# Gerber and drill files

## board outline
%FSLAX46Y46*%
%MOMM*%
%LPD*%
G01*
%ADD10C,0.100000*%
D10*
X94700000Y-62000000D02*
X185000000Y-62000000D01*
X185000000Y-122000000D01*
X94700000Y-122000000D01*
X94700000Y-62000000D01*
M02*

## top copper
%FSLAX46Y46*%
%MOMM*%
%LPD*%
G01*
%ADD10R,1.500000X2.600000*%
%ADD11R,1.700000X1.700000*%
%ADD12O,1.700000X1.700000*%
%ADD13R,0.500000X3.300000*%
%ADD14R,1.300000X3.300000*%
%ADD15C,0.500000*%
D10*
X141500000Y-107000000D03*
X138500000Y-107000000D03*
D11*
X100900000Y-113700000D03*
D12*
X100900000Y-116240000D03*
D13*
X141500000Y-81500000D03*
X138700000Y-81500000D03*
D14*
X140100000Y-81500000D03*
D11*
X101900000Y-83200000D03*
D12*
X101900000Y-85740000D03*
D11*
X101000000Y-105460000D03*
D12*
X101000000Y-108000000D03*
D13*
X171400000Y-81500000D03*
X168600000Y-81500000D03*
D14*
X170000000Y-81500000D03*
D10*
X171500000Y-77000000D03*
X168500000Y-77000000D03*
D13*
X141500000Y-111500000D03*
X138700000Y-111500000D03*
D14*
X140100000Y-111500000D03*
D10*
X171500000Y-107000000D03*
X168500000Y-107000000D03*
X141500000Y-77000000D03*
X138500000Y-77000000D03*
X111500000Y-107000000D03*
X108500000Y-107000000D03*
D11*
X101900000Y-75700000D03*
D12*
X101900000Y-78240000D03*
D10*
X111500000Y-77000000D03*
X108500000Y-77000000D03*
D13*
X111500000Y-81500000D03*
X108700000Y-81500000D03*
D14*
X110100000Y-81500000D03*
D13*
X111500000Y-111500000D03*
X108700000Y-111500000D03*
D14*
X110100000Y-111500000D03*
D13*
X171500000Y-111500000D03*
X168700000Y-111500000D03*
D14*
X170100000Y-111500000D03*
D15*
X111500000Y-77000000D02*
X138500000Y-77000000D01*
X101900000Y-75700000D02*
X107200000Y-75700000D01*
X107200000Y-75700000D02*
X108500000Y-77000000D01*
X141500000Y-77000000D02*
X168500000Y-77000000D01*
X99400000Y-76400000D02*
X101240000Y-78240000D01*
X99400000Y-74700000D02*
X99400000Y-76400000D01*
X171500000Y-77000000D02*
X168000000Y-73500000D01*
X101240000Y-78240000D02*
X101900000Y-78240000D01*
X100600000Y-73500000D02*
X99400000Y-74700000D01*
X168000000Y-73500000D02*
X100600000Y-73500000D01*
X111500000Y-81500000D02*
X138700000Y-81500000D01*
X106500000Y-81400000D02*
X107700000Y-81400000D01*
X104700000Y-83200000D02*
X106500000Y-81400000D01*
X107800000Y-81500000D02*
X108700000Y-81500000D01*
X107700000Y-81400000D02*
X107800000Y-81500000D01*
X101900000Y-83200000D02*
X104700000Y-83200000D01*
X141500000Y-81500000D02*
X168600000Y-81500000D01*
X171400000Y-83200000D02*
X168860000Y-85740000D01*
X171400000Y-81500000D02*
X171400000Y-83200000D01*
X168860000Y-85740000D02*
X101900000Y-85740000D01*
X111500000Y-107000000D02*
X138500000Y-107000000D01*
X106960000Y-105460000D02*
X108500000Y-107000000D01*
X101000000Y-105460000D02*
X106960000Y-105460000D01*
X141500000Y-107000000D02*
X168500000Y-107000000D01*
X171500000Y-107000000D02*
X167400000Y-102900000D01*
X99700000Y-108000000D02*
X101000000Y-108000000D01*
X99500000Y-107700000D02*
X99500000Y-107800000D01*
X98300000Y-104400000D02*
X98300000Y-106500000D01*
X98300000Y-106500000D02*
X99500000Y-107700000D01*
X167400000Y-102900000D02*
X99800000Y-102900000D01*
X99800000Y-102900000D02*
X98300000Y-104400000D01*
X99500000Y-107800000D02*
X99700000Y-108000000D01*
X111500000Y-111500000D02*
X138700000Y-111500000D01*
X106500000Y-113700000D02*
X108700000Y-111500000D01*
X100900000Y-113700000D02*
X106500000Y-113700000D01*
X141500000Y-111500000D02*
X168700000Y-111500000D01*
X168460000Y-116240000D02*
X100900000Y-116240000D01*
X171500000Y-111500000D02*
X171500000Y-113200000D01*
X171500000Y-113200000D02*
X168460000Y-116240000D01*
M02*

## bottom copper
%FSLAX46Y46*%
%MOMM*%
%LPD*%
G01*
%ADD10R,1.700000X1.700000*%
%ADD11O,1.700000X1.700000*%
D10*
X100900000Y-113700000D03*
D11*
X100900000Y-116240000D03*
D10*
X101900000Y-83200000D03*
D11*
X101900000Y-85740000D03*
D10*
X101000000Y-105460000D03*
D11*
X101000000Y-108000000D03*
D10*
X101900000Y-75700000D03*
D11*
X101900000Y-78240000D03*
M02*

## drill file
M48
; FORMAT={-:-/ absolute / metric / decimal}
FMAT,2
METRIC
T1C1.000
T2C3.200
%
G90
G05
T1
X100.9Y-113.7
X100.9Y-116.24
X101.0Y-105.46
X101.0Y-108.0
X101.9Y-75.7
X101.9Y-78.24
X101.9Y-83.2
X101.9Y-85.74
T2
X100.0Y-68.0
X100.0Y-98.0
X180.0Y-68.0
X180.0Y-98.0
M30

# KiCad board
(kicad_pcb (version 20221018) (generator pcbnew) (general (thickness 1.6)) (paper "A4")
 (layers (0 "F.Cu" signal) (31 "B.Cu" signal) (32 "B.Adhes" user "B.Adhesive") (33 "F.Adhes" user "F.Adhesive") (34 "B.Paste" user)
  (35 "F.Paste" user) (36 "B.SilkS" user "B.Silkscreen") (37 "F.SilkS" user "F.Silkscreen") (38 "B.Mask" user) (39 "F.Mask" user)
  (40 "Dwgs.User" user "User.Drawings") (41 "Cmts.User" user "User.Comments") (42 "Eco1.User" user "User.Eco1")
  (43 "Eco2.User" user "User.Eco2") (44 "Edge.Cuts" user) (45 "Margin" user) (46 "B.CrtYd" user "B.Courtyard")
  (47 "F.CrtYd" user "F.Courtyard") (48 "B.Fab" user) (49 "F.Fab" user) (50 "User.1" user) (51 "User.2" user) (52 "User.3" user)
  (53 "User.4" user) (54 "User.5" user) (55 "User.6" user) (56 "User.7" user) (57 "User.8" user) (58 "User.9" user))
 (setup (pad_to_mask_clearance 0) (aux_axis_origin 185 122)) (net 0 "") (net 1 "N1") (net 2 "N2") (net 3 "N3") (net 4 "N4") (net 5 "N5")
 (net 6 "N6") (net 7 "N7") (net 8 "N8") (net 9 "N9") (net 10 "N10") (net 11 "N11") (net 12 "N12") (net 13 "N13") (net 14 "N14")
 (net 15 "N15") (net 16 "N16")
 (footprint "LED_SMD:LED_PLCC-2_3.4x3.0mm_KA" (layer "F.Cu") (at 140 107 180)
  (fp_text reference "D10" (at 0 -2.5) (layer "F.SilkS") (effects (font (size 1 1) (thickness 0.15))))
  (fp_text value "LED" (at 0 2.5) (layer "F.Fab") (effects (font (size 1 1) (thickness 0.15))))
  (pad "1" smd rect (at -1.5 0 180) (size 1.5 2.6) (layers "F.Cu" "F.Paste" "F.Mask") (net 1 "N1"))
  (pad "2" smd rect (at 1.5 0 180) (size 1.5 2.6) (layers "F.Cu" "F.Paste" "F.Mask") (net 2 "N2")))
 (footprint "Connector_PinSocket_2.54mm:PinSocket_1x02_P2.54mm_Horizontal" (layer "F.Cu") (at 100.9 113.7)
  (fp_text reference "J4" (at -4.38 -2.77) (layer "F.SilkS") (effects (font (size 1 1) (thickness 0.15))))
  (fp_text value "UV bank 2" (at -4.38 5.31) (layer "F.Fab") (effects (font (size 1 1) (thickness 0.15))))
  (pad "1" thru_hole rect (at 0 0) (size 1.7 1.7) (drill 1) (layers "*.Cu" "*.Mask") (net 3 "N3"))
  (pad "2" thru_hole oval (at 0 2.54) (size 1.7 1.7) (drill 1) (layers "*.Cu" "*.Mask") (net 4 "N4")))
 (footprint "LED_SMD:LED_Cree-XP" (layer "F.Cu") (at 140.1 81.5 180)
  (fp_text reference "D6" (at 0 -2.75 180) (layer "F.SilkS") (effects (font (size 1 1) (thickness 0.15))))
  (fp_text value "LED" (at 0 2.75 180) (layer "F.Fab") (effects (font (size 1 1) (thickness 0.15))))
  (pad "" smd rect (at 0 -1 180) (size 1.01 0.75) (layers "F.Paste"))
  (pad "" smd rect (at 0 0 180) (size 1.01 0.75) (layers "F.Paste"))
  (pad "" smd rect (at 0 1 180) (size 1.01 0.75) (layers "F.Paste"))
  (pad "1" smd rect (at -1.4 0 180) (size 0.5 3.3) (layers "F.Cu" "F.Paste" "F.Mask") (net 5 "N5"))
  (pad "2" smd rect (at 1.4 0 180) (size 0.5 3.3) (layers "F.Cu" "F.Paste" "F.Mask") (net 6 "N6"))
  (pad "3" smd rect (at 0 0 180) (size 1.3 3.3) (layers "F.Cu" "F.Mask")))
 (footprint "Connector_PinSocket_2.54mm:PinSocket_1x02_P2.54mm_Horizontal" (layer "F.Cu") (at 101.9 83.2)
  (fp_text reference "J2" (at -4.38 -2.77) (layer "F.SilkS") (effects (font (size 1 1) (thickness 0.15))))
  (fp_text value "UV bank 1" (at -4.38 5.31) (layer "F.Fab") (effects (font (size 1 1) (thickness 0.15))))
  (pad "1" thru_hole rect (at 0 0) (size 1.7 1.7) (drill 1) (layers "*.Cu" "*.Mask") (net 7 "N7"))
  (pad "2" thru_hole oval (at 0 2.54) (size 1.7 1.7) (drill 1) (layers "*.Cu" "*.Mask") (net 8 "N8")))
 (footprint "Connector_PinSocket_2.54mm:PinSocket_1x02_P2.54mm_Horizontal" (layer "F.Cu") (at 101 105.46)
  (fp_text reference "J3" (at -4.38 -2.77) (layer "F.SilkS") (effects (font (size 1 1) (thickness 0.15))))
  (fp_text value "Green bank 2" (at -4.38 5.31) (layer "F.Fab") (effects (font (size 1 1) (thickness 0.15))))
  (pad "1" thru_hole rect (at 0 0) (size 1.7 1.7) (drill 1) (layers "*.Cu" "*.Mask") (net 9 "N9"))
  (pad "2" thru_hole oval (at 0 2.54) (size 1.7 1.7) (drill 1) (layers "*.Cu" "*.Mask") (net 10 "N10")))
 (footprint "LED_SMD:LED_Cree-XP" (layer "F.Cu") (at 170 81.5 180)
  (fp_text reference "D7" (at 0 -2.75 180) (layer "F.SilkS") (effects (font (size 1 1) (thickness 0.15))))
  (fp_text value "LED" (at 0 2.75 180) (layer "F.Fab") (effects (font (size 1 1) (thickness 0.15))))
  (pad "" smd rect (at 0 -1 180) (size 1.01 0.75) (layers "F.Paste"))
  (pad "" smd rect (at 0 0 180) (size 1.01 0.75) (layers "F.Paste"))
  (pad "" smd rect (at 0 1 180) (size 1.01 0.75) (layers "F.Paste"))
  (pad "1" smd rect (at -1.4 0 180) (size 0.5 3.3) (layers "F.Cu" "F.Paste" "F.Mask") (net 8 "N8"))
  (pad "2" smd rect (at 1.4 0 180) (size 0.5 3.3) (layers "F.Cu" "F.Paste" "F.Mask") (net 5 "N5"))
  (pad "3" smd rect (at 0 0 180) (size 1.3 3.3) (layers "F.Cu" "F.Mask")))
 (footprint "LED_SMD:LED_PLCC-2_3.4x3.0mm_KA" (layer "F.Cu") (at 170 77 180)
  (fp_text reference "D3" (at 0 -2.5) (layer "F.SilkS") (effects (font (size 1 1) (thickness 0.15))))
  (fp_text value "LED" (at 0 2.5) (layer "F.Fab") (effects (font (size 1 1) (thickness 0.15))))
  (pad "1" smd rect (at -1.5 0 180) (size 1.5 2.6) (layers "F.Cu" "F.Paste" "F.Mask") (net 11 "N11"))
  (pad "2" smd rect (at 1.5 0 180) (size 1.5 2.6) (layers "F.Cu" "F.Paste" "F.Mask") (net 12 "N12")))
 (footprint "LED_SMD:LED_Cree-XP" (layer "F.Cu") (at 140.1 111.5 180)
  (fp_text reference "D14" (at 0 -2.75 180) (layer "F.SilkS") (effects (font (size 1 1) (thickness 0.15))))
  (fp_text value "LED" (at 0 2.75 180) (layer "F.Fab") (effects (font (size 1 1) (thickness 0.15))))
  (pad "" smd rect (at 0 -1 180) (size 1.01 0.75) (layers "F.Paste"))
  (pad "" smd rect (at 0 0 180) (size 1.01 0.75) (layers "F.Paste"))
  (pad "" smd rect (at 0 1 180) (size 1.01 0.75) (layers "F.Paste"))
  (pad "1" smd rect (at -1.4 0 180) (size 0.5 3.3) (layers "F.Cu" "F.Paste" "F.Mask") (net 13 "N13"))
  (pad "2" smd rect (at 1.4 0 180) (size 0.5 3.3) (layers "F.Cu" "F.Paste" "F.Mask") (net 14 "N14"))
  (pad "3" smd rect (at 0 0 180) (size 1.3 3.3) (layers "F.Cu" "F.Mask")))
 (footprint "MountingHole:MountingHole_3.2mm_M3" (layer "F.Cu") (at 180 68)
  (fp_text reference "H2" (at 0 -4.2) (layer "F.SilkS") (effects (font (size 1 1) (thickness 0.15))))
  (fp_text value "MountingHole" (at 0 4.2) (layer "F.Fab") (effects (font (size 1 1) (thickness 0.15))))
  (pad "" np_thru_hole circle (at 0 0) (size 3.2 3.2) (drill 3.2) (layers "*.Cu" "*.Mask")))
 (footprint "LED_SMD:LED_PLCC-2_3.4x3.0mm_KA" (layer "F.Cu") (at 170 107 180)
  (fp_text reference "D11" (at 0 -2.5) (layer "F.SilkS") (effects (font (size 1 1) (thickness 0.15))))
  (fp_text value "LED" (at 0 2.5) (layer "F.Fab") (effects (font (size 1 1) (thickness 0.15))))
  (pad "1" smd rect (at -1.5 0 180) (size 1.5 2.6) (layers "F.Cu" "F.Paste" "F.Mask") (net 10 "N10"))
  (pad "2" smd rect (at 1.5 0 180) (size 1.5 2.6) (layers "F.Cu" "F.Paste" "F.Mask") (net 1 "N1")))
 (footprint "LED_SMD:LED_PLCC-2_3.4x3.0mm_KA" (layer "F.Cu") (at 140 77 180)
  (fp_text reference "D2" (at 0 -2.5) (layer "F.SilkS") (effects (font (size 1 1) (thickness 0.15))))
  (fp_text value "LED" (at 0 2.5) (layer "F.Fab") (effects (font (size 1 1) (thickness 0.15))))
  (pad "1" smd rect (at -1.5 0 180) (size 1.5 2.6) (layers "F.Cu" "F.Paste" "F.Mask") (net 12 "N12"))
  (pad "2" smd rect (at 1.5 0 180) (size 1.5 2.6) (layers "F.Cu" "F.Paste" "F.Mask") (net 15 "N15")))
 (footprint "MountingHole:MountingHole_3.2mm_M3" (layer "F.Cu") (at 100 98)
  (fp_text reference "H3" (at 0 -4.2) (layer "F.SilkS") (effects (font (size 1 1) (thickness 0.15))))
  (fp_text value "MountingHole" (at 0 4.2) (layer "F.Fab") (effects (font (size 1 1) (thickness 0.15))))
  (pad "" np_thru_hole circle (at 0 0) (size 3.2 3.2) (drill 3.2) (layers "*.Cu" "*.Mask")))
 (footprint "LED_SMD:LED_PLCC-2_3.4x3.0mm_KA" (layer "F.Cu") (at 110 107 180)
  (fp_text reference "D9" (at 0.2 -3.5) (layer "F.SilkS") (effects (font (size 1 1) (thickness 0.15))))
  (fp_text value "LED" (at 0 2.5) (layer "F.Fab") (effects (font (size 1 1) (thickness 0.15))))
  (pad "1" smd rect (at -1.5 0 180) (size 1.5 2.6) (layers "F.Cu" "F.Paste" "F.Mask") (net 2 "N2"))
  (pad "2" smd rect (at 1.5 0 180) (size 1.5 2.6) (layers "F.Cu" "F.Paste" "F.Mask") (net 9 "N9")))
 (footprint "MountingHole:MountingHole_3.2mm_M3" (layer "F.Cu") (at 180 98)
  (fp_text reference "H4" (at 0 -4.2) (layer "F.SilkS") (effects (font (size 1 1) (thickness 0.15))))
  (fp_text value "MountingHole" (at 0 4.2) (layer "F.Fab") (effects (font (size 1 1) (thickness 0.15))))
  (pad "" np_thru_hole circle (at 0 0) (size 3.2 3.2) (drill 3.2) (layers "*.Cu" "*.Mask")))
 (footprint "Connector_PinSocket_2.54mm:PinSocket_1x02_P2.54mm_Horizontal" (layer "F.Cu") (at 101.9 75.7)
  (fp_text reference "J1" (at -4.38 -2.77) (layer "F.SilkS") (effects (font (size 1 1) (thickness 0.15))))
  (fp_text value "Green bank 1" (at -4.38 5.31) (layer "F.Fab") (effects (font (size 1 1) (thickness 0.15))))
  (pad "1" thru_hole rect (at 0 0) (size 1.7 1.7) (drill 1) (layers "*.Cu" "*.Mask") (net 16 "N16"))
  (pad "2" thru_hole oval (at 0 2.54) (size 1.7 1.7) (drill 1) (layers "*.Cu" "*.Mask") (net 11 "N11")))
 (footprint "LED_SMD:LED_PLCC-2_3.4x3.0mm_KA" (layer "F.Cu") (at 110 77 180)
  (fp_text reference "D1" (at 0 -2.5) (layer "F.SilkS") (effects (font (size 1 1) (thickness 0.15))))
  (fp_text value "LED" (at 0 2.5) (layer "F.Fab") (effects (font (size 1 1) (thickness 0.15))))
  (pad "1" smd rect (at -1.5 0 180) (size 1.5 2.6) (layers "F.Cu" "F.Paste" "F.Mask") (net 15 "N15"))
  (pad "2" smd rect (at 1.5 0 180) (size 1.5 2.6) (layers "F.Cu" "F.Paste" "F.Mask") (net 16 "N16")))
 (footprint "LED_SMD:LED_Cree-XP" (layer "F.Cu") (at 110.1 81.5 180)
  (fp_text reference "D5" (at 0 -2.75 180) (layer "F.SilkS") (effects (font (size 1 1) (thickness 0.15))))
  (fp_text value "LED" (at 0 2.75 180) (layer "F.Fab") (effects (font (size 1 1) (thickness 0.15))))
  (pad "" smd rect (at 0 -1 180) (size 1.01 0.75) (layers "F.Paste"))
  (pad "" smd rect (at 0 0 180) (size 1.01 0.75) (layers "F.Paste"))
  (pad "" smd rect (at 0 1 180) (size 1.01 0.75) (layers "F.Paste"))
  (pad "1" smd rect (at -1.4 0 180) (size 0.5 3.3) (layers "F.Cu" "F.Paste" "F.Mask") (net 6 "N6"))
  (pad "2" smd rect (at 1.4 0 180) (size 0.5 3.3) (layers "F.Cu" "F.Paste" "F.Mask") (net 7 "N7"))
  (pad "3" smd rect (at 0 0 180) (size 1.3 3.3) (layers "F.Cu" "F.Mask")))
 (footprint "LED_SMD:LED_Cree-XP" (layer "F.Cu") (at 110.1 111.5 180)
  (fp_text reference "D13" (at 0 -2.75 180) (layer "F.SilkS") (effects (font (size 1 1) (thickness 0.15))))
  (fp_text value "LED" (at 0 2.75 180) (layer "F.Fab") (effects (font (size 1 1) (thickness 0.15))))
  (pad "" smd rect (at 0 -1 180) (size 1.01 0.75) (layers "F.Paste"))
  (pad "" smd rect (at 0 0 180) (size 1.01 0.75) (layers "F.Paste"))
  (pad "" smd rect (at 0 1 180) (size 1.01 0.75) (layers "F.Paste"))
  (pad "1" smd rect (at -1.4 0 180) (size 0.5 3.3) (layers "F.Cu" "F.Paste" "F.Mask") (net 14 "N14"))
  (pad "2" smd rect (at 1.4 0 180) (size 0.5 3.3) (layers "F.Cu" "F.Paste" "F.Mask") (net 3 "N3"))
  (pad "3" smd rect (at 0 0 180) (size 1.3 3.3) (layers "F.Cu" "F.Mask")))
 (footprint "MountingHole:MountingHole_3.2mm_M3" (layer "F.Cu") (at 100 68)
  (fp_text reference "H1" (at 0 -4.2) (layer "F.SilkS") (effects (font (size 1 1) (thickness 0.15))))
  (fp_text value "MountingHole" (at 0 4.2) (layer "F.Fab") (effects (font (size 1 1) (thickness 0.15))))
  (pad "" np_thru_hole circle (at 0 0) (size 3.2 3.2) (drill 3.2) (layers "*.Cu" "*.Mask")))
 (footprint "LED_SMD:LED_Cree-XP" (layer "F.Cu") (at 170.1 111.5 180)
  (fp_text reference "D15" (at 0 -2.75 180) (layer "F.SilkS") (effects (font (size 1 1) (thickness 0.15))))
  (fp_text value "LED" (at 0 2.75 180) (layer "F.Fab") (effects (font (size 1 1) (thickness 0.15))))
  (pad "" smd rect (at 0 -1 180) (size 1.01 0.75) (layers "F.Paste"))
  (pad "" smd rect (at 0 0 180) (size 1.01 0.75) (layers "F.Paste"))
  (pad "" smd rect (at 0 1 180) (size 1.01 0.75) (layers "F.Paste"))
  (pad "1" smd rect (at -1.4 0 180) (size 0.5 3.3) (layers "F.Cu" "F.Paste" "F.Mask") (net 4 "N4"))
  (pad "2" smd rect (at 1.4 0 180) (size 0.5 3.3) (layers "F.Cu" "F.Paste" "F.Mask") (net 13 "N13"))
  (pad "3" smd rect (at 0 0 180) (size 1.3 3.3) (layers "F.Cu" "F.Mask")))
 (gr_rect (start 94.7 62) (end 185 122) (stroke (width 0.1) (type default)) (fill none) (layer "Edge.Cuts"))
 (segment (start 111.5 77) (end 138.5 77) (width 0.5) (layer "F.Cu") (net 15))
 (segment (start 101.9 75.7) (end 107.2 75.7) (width 0.5) (layer "F.Cu") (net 16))
 (segment (start 107.2 75.7) (end 108.5 77) (width 0.5) (layer "F.Cu") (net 16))
 (segment (start 141.5 77) (end 168.5 77) (width 0.5) (layer "F.Cu") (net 12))
 (segment (start 99.4 76.4) (end 101.24 78.24) (width 0.5) (layer "F.Cu") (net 11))
 (segment (start 99.4 74.7) (end 99.4 76.4) (width 0.5) (layer "F.Cu") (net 11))
 (segment (start 171.5 77) (end 168 73.5) (width 0.5) (layer "F.Cu") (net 11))
 (segment (start 101.24 78.24) (end 101.9 78.24) (width 0.5) (layer "F.Cu") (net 11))
 (segment (start 100.6 73.5) (end 99.4 74.7) (width 0.5) (layer "F.Cu") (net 11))
 (segment (start 168 73.5) (end 100.6 73.5) (width 0.5) (layer "F.Cu") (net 11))
 (segment (start 111.5 81.5) (end 138.7 81.5) (width 0.5) (layer "F.Cu") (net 6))
 (segment (start 106.5 81.4) (end 107.7 81.4) (width 0.5) (layer "F.Cu") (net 7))
 (segment (start 104.7 83.2) (end 106.5 81.4) (width 0.5) (layer "F.Cu") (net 7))
 (segment (start 107.8 81.5) (end 108.7 81.5) (width 0.5) (layer "F.Cu") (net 7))
 (segment (start 107.7 81.4) (end 107.8 81.5) (width 0.5) (layer "F.Cu") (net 7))
 (segment (start 101.9 83.2) (end 104.7 83.2) (width 0.5) (layer "F.Cu") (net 7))
 (segment (start 141.5 81.5) (end 168.6 81.5) (width 0.5) (layer "F.Cu") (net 5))
 (segment (start 171.4 83.2) (end 168.86 85.74) (width 0.5) (layer "F.Cu") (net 8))
 (segment (start 171.4 81.5) (end 171.4 83.2) (width 0.5) (layer "F.Cu") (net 8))
 (segment (start 168.86 85.74) (end 101.9 85.74) (width 0.5) (layer "F.Cu") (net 8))
 (segment (start 111.5 107) (end 138.5 107) (width 0.5) (layer "F.Cu") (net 2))
 (segment (start 106.96 105.46) (end 108.5 107) (width 0.5) (layer "F.Cu") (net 9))
 (segment (start 101 105.46) (end 106.96 105.46) (width 0.5) (layer "F.Cu") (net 9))
 (segment (start 141.5 107) (end 168.5 107) (width 0.5) (layer "F.Cu") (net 1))
 (segment (start 171.5 107) (end 167.4 102.9) (width 0.5) (layer "F.Cu") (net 10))
 (segment (start 99.7 108) (end 101 108) (width 0.5) (layer "F.Cu") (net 10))
 (segment (start 99.5 107.7) (end 99.5 107.8) (width 0.5) (layer "F.Cu") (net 10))
 (segment (start 98.3 104.4) (end 98.3 106.5) (width 0.5) (layer "F.Cu") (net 10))
 (segment (start 98.3 106.5) (end 99.5 107.7) (width 0.5) (layer "F.Cu") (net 10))
 (segment (start 167.4 102.9) (end 99.8 102.9) (width 0.5) (layer "F.Cu") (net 10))
 (segment (start 99.8 102.9) (end 98.3 104.4) (width 0.5) (layer "F.Cu") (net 10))
 (segment (start 99.5 107.8) (end 99.7 108) (width 0.5) (layer "F.Cu") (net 10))
 (segment (start 111.5 111.5) (end 138.7 111.5) (width 0.5) (layer "F.Cu") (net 14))
 (segment (start 106.5 113.7) (end 108.7 111.5) (width 0.5) (layer "F.Cu") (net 3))
 (segment (start 100.9 113.7) (end 106.5 113.7) (width 0.5) (layer "F.Cu") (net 3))
 (segment (start 141.5 111.5) (end 168.7 111.5) (width 0.5) (layer "F.Cu") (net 13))
 (segment (start 168.46 116.24) (end 100.9 116.24) (width 0.5) (layer "F.Cu") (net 4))
 (segment (start 171.5 111.5) (end 171.5 113.2) (width 0.5) (layer "F.Cu") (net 4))
 (segment (start 171.5 113.2) (end 168.46 116.24) (width 0.5) (layer "F.Cu") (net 4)))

